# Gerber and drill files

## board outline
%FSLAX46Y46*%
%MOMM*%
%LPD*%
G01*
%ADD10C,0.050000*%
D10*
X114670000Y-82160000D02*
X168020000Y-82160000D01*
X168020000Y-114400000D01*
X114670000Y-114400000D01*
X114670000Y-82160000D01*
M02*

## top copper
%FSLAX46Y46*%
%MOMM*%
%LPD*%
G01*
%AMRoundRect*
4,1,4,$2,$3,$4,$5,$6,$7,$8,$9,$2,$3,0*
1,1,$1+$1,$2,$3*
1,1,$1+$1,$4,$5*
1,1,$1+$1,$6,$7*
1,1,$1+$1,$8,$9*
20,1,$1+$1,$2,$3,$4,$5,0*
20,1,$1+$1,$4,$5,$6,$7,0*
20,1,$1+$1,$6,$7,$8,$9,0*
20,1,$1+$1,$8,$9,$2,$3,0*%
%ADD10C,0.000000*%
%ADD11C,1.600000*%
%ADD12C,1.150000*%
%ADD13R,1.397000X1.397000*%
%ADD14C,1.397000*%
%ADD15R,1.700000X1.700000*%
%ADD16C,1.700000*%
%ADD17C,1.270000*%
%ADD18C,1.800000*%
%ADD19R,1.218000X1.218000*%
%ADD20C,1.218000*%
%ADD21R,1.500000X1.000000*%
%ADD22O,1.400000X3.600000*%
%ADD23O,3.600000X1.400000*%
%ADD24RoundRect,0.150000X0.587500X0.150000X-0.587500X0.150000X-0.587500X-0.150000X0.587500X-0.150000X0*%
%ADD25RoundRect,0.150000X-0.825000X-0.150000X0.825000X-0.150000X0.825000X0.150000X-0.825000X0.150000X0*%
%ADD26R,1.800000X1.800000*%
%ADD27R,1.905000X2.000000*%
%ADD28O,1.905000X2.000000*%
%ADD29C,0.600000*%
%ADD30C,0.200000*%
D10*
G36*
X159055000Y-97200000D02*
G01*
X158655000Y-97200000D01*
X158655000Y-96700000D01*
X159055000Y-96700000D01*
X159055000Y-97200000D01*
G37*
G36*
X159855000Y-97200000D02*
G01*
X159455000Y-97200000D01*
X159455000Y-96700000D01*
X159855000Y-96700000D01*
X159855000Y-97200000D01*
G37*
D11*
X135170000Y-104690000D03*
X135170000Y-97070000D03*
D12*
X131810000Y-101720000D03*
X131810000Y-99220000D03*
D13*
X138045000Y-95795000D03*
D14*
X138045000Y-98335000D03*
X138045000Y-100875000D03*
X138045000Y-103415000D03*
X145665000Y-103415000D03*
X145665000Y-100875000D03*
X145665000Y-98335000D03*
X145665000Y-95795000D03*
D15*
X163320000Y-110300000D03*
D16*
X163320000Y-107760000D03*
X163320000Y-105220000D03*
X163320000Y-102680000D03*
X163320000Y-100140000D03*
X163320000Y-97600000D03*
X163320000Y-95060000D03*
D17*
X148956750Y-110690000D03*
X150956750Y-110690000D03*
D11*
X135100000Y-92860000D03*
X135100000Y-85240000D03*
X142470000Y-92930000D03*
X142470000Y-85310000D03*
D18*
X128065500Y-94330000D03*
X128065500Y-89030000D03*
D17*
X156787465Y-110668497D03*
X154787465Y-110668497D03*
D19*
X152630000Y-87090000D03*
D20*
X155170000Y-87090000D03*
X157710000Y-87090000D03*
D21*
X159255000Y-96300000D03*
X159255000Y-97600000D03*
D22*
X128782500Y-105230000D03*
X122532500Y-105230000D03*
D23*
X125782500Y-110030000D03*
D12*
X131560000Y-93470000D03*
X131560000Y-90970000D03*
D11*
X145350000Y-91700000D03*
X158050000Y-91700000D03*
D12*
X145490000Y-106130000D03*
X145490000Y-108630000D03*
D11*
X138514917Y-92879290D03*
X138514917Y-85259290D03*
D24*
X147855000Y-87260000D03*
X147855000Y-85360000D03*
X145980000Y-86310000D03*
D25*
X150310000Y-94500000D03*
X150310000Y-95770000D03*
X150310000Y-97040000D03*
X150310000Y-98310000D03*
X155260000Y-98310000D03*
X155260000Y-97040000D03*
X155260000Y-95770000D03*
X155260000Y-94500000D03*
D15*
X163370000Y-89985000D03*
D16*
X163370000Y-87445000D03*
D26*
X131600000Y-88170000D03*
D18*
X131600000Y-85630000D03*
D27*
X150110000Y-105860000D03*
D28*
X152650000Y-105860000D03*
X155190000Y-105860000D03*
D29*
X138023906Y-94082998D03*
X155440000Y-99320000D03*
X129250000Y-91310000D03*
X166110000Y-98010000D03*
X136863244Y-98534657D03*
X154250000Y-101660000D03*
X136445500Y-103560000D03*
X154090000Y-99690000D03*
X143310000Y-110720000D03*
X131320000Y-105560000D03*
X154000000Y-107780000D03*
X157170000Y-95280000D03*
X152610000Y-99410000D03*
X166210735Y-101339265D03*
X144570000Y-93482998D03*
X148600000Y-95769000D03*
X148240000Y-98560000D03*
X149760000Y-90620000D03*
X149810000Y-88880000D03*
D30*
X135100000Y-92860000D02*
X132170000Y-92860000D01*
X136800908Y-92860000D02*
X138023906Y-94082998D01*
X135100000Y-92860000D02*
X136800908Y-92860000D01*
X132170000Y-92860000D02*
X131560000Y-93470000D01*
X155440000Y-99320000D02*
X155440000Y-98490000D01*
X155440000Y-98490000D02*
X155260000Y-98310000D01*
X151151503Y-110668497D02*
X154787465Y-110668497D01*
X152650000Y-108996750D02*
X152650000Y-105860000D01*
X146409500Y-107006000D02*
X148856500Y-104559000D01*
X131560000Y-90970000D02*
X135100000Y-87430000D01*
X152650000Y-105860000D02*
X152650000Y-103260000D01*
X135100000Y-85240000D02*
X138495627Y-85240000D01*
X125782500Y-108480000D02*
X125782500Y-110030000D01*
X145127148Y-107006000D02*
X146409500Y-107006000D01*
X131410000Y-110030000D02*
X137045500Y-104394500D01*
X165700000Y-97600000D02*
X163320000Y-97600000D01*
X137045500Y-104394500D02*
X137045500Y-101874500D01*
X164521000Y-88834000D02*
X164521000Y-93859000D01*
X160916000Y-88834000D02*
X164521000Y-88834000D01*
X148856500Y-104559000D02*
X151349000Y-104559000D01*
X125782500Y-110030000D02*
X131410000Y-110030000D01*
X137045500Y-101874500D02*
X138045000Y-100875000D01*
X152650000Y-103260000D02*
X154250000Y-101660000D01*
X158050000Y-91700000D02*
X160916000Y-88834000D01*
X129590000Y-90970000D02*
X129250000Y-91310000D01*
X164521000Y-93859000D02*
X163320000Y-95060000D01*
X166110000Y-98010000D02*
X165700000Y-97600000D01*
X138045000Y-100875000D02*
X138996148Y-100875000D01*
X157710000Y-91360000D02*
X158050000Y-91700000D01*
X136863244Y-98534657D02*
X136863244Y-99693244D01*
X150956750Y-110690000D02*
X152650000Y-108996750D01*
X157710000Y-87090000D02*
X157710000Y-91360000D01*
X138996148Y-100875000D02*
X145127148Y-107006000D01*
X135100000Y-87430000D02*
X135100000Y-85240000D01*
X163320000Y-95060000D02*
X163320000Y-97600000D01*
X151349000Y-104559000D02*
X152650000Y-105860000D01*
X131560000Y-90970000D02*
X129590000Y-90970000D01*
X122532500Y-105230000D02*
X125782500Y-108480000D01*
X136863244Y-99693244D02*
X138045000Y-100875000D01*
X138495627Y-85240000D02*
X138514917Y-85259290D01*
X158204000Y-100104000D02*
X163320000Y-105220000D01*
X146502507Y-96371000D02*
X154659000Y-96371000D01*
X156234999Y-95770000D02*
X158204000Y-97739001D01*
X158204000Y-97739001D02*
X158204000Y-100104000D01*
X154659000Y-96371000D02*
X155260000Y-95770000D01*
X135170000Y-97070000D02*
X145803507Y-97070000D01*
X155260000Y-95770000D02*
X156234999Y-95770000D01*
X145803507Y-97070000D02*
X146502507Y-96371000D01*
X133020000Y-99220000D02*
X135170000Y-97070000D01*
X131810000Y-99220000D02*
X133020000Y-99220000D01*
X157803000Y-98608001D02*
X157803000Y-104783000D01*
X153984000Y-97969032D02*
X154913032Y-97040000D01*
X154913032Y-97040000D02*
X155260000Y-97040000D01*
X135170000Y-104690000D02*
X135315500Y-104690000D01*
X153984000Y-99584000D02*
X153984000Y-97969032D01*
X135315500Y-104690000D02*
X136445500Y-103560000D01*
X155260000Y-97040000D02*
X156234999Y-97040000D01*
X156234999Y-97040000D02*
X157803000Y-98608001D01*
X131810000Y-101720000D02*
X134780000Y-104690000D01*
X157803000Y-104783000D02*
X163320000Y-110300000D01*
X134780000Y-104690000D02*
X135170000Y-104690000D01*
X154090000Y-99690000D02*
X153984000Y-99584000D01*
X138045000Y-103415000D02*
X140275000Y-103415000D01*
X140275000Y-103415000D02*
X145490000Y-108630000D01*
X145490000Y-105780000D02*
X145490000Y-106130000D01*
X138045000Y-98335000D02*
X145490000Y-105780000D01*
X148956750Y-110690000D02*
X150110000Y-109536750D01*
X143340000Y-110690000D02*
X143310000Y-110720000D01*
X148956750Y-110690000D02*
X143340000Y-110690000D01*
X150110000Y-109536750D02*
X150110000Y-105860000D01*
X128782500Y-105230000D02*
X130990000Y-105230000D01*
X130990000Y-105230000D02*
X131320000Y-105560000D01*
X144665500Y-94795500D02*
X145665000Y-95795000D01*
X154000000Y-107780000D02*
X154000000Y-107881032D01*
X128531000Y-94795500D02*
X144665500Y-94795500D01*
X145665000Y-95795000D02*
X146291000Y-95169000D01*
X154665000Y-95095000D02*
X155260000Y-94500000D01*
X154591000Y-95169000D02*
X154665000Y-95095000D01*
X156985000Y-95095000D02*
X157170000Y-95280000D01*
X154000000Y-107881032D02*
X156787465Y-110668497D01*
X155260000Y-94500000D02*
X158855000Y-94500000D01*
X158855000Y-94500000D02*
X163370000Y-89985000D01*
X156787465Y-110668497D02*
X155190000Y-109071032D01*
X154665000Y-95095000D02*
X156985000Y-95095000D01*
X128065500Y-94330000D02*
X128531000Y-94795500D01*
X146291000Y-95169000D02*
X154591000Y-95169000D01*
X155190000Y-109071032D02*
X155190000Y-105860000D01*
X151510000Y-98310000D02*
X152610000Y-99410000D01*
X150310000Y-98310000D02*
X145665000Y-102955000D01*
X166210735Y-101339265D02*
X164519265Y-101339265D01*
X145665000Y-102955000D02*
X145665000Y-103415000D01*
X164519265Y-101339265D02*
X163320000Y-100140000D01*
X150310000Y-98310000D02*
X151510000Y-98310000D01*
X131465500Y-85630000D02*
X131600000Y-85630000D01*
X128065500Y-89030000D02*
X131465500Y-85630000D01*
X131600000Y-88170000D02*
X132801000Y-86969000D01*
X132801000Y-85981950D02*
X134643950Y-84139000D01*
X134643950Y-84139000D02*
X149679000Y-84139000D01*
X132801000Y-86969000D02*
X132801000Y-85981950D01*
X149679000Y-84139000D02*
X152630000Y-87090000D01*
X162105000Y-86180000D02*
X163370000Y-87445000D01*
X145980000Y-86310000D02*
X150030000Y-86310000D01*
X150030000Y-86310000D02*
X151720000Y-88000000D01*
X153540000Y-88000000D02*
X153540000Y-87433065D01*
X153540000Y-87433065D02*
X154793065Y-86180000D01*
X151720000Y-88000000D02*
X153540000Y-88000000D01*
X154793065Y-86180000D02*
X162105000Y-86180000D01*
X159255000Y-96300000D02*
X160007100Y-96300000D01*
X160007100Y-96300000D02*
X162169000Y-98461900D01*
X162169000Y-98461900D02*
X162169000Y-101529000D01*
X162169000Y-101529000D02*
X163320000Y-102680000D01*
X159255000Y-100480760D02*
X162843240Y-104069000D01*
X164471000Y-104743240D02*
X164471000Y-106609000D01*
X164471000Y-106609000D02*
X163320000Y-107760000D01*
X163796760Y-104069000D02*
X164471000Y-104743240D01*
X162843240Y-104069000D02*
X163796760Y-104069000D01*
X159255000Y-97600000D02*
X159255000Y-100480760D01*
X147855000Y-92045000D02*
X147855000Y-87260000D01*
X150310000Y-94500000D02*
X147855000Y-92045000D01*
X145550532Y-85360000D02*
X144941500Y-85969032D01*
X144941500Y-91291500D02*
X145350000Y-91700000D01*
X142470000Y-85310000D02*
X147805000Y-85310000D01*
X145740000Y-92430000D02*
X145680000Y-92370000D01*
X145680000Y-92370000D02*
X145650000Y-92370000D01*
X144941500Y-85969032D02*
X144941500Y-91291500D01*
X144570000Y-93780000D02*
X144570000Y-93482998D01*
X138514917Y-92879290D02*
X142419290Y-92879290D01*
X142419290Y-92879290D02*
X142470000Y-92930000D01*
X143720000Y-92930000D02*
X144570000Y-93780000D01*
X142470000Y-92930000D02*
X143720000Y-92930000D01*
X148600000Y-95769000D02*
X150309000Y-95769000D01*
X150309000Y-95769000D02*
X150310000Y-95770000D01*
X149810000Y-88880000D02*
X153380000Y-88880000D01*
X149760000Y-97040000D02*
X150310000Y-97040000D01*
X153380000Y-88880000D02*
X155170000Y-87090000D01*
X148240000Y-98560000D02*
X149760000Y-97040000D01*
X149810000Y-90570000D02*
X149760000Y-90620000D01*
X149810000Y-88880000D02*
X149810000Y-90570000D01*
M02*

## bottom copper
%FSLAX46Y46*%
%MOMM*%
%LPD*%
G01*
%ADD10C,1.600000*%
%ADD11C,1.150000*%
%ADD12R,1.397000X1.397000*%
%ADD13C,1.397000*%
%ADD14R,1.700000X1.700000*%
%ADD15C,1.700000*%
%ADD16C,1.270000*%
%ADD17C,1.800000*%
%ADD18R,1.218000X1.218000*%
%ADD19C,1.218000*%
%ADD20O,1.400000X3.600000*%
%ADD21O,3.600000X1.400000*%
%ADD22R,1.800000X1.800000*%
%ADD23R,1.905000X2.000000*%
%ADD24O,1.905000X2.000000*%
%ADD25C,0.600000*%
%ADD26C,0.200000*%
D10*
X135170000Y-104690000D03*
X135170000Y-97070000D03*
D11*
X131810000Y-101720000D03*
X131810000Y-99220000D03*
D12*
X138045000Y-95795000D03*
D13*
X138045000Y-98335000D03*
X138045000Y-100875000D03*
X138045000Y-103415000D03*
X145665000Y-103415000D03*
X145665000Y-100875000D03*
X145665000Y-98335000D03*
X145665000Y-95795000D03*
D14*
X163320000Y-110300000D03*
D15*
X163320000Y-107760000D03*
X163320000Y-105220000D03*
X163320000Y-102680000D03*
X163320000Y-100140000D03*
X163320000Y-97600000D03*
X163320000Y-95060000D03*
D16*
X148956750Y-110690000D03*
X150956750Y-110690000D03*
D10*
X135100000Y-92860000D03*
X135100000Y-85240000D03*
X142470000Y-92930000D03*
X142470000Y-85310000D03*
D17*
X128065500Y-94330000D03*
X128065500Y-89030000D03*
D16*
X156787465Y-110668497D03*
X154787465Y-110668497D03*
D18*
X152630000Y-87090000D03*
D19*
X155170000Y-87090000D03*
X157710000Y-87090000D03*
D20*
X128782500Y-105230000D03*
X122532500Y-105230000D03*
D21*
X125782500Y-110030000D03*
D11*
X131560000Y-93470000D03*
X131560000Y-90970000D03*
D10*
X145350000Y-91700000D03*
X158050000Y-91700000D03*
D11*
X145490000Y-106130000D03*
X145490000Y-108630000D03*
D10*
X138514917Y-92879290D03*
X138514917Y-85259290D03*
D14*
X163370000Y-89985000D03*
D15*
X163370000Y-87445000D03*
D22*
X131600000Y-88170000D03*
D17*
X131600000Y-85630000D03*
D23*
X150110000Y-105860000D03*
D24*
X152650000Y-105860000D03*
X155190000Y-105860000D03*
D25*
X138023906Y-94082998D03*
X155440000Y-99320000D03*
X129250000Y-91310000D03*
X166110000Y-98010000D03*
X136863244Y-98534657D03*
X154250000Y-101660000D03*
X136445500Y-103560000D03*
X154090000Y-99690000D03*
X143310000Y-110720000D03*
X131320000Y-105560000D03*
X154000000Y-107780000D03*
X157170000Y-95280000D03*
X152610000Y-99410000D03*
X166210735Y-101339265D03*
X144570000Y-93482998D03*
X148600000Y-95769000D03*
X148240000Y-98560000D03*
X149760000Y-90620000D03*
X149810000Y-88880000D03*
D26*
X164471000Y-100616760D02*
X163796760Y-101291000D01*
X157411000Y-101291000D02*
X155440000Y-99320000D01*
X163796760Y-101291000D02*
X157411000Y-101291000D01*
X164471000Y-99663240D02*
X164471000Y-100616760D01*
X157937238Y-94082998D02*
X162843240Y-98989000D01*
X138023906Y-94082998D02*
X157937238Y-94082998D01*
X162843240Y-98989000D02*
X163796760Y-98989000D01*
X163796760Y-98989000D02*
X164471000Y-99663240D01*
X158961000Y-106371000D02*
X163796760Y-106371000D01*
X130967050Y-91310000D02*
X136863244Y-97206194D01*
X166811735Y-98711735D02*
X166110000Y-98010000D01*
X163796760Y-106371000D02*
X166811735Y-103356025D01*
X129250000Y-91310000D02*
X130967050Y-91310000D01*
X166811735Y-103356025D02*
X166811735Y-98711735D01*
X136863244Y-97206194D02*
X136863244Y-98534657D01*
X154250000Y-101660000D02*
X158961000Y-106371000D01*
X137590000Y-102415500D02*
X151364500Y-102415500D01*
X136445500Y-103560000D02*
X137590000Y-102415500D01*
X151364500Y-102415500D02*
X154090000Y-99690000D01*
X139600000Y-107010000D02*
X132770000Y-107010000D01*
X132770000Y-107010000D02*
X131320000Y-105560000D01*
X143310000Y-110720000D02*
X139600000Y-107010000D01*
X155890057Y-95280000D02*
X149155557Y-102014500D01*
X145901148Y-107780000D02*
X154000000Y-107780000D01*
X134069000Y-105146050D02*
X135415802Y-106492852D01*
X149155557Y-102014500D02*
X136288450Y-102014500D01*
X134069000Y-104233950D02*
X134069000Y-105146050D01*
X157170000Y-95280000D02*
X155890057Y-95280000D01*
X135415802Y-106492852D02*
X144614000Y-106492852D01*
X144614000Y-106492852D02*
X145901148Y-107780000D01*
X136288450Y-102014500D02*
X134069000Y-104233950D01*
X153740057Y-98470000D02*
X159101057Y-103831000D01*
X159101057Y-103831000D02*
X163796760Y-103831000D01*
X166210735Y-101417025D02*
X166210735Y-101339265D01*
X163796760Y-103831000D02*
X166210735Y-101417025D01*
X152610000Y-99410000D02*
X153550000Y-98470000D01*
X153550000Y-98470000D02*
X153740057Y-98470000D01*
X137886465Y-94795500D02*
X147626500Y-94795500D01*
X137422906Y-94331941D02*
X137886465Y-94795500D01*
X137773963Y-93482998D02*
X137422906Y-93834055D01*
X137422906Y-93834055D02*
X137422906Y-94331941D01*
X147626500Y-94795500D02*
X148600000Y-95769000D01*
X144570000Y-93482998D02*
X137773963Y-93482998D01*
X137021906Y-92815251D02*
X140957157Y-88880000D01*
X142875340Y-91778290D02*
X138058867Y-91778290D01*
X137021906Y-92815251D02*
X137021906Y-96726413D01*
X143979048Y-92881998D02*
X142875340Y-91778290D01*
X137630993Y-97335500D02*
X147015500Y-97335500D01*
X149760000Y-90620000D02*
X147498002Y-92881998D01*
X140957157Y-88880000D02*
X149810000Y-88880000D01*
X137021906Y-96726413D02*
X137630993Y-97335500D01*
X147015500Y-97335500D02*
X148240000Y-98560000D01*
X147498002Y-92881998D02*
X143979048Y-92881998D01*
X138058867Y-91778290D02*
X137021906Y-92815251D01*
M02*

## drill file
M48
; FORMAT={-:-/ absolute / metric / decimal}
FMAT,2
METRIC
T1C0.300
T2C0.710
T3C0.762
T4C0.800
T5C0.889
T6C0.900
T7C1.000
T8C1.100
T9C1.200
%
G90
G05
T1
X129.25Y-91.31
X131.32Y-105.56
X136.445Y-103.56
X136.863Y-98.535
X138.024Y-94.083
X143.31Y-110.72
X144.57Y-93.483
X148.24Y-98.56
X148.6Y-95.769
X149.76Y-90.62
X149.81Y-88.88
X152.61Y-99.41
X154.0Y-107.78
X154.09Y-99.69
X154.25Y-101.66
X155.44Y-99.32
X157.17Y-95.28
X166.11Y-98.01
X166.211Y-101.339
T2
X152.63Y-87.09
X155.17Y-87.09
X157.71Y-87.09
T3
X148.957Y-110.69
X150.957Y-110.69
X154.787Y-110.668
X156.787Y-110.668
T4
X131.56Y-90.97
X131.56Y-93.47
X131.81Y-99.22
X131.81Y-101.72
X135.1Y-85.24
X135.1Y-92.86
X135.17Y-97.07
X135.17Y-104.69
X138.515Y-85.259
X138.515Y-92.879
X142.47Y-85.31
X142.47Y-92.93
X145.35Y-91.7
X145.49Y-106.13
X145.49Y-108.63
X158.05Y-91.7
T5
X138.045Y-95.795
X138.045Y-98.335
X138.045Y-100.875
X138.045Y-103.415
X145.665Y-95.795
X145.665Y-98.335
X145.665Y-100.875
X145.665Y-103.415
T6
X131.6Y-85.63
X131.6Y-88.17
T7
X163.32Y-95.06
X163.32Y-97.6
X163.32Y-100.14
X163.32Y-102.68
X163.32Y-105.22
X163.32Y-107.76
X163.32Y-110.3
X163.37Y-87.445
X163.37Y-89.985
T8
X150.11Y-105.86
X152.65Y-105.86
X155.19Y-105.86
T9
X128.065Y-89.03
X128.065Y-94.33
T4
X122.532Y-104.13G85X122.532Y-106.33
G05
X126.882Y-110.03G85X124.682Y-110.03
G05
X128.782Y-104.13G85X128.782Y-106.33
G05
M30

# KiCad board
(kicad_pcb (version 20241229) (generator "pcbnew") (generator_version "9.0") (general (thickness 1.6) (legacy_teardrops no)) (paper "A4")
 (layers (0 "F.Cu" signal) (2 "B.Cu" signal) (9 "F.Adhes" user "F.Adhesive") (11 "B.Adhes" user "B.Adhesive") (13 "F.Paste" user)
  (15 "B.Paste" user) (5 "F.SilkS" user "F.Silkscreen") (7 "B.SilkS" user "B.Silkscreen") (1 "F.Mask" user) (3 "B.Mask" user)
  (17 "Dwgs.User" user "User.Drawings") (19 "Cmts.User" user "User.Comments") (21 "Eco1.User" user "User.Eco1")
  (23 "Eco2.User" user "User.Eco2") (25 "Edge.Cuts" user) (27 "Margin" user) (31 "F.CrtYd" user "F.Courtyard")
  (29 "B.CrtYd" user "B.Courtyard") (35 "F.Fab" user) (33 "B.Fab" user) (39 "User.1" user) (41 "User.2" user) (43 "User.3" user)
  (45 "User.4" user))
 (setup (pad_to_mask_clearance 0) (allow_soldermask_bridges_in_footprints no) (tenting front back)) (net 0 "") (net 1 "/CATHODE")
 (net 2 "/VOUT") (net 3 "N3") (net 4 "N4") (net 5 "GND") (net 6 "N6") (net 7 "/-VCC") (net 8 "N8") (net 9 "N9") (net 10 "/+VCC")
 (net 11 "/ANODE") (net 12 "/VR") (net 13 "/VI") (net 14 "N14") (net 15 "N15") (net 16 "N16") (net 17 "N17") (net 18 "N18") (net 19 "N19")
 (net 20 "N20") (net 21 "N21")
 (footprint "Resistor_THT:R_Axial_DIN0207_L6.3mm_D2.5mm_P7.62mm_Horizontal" (layer "F.Cu") (at 135.17 104.69 90)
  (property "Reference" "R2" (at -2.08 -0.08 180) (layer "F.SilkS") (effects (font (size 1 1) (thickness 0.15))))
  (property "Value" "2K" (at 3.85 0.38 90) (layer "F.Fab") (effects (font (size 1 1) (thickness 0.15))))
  (pad "1" thru_hole circle (at 0 0 90) (size 1.6 1.6) (drill 0.8) (layers "*.Cu" "*.Mask") (remove_unused_layers no) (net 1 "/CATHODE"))
  (pad "2" thru_hole circle (at 7.62 0 90) (size 1.6 1.6) (drill 0.8) (layers "*.Cu" "*.Mask") (remove_unused_layers no) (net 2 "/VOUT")))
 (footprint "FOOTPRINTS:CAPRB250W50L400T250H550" (layer "F.Cu") (at 131.81 100.47 90)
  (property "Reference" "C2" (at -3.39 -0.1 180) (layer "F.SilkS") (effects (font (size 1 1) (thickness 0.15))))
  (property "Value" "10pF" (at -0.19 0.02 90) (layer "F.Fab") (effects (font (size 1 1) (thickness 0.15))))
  (pad "1" thru_hole circle (at -1.25 0 90) (size 1.15 1.15) (drill 0.8) (layers "*.Cu" "*.Mask") (remove_unused_layers no)
   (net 1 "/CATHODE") (solder_mask_margin 0.102))
  (pad "2" thru_hole circle (at 1.25 0 90) (size 1.15 1.15) (drill 0.8) (layers "*.Cu" "*.Mask") (remove_unused_layers no) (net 2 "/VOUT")
   (solder_mask_margin 0.102)))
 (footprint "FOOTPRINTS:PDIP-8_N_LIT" (layer "F.Cu") (at 138.045 95.795)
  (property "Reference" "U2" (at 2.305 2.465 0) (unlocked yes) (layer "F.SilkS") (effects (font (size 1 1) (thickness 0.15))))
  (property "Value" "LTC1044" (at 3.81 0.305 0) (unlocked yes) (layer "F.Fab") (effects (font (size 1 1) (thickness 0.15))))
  (pad "1" thru_hole rect (at 0 0) (size 1.397 1.397) (drill 0.889) (layers "*.Cu" "*.Mask") (remove_unused_layers no) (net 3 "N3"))
  (pad "2" thru_hole circle (at 0 2.54) (size 1.397 1.397) (drill 0.889) (layers "*.Cu" "*.Mask") (remove_unused_layers no) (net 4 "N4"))
  (pad "3" thru_hole circle (at 0 5.08) (size 1.397 1.397) (drill 0.889) (layers "*.Cu" "*.Mask") (remove_unused_layers no) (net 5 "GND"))
  (pad "4" thru_hole circle (at 0 7.62) (size 1.397 1.397) (drill 0.889) (layers "*.Cu" "*.Mask") (remove_unused_layers no) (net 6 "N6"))
  (pad "5" thru_hole circle (at 7.62 7.62) (size 1.397 1.397) (drill 0.889) (layers "*.Cu" "*.Mask") (remove_unused_layers no)
   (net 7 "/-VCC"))
  (pad "6" thru_hole circle (at 7.62 5.08) (size 1.397 1.397) (drill 0.889) (layers "*.Cu" "*.Mask") (remove_unused_layers no) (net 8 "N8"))
  (pad "7" thru_hole circle (at 7.62 2.54) (size 1.397 1.397) (drill 0.889) (layers "*.Cu" "*.Mask") (remove_unused_layers no) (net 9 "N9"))
  (pad "8" thru_hole circle (at 7.62 0) (size 1.397 1.397) (drill 0.889) (layers "*.Cu" "*.Mask") (remove_unused_layers no) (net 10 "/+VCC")))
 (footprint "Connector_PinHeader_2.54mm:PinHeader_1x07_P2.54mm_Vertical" (layer "F.Cu") (at 163.32 110.3 180)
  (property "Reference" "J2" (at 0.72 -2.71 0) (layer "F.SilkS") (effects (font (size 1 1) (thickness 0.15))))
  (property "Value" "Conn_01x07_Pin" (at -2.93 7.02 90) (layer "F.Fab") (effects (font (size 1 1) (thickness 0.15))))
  (pad "1" thru_hole rect (at 0 0 180) (size 1.7 1.7) (drill 1) (layers "*.Cu" "*.Mask") (remove_unused_layers no) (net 1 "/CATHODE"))
  (pad "2" thru_hole circle (at 0 2.54 180) (size 1.7 1.7) (drill 1) (layers "*.Cu" "*.Mask") (remove_unused_layers no) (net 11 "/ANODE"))
  (pad "3" thru_hole circle (at 0 5.08 180) (size 1.7 1.7) (drill 1) (layers "*.Cu" "*.Mask") (remove_unused_layers no) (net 2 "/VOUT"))
  (pad "4" thru_hole circle (at 0 7.62 180) (size 1.7 1.7) (drill 1) (layers "*.Cu" "*.Mask") (remove_unused_layers no) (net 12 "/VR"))
  (pad "5" thru_hole circle (at 0 10.16 180) (size 1.7 1.7) (drill 1) (layers "*.Cu" "*.Mask") (remove_unused_layers no) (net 7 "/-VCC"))
  (pad "6" thru_hole circle (at 0 12.7 180) (size 1.7 1.7) (drill 1) (layers "*.Cu" "*.Mask") (remove_unused_layers no) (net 5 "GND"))
  (pad "7" thru_hole circle (at 0 15.24 180) (size 1.7 1.7) (drill 1) (layers "*.Cu" "*.Mask") (remove_unused_layers no) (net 5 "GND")))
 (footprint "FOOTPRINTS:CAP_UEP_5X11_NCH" (layer "F.Cu") (at 148.95675 110.69)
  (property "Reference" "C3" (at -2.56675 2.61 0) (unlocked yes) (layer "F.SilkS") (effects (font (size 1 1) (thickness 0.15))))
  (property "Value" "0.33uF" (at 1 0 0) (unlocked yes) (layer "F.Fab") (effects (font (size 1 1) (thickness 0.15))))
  (pad "1" thru_hole circle (at 0 0) (size 1.27 1.27) (drill 0.762) (layers "*.Cu" "*.Mask") (remove_unused_layers no) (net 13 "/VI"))
  (pad "2" thru_hole circle (at 2 0) (size 1.27 1.27) (drill 0.762) (layers "*.Cu" "*.Mask") (remove_unused_layers no) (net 5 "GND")))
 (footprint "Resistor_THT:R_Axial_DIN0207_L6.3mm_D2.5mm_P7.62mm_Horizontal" (layer "F.Cu") (at 135.1 92.86 90)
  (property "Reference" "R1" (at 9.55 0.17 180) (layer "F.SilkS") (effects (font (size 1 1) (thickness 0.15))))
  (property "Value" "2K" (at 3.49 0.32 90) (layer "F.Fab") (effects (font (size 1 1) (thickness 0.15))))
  (pad "1" thru_hole circle (at 0 0 90) (size 1.6 1.6) (drill 0.8) (layers "*.Cu" "*.Mask") (remove_unused_layers no) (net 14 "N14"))
  (pad "2" thru_hole circle (at 7.62 0 90) (size 1.6 1.6) (drill 0.8) (layers "*.Cu" "*.Mask") (remove_unused_layers no) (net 5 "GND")))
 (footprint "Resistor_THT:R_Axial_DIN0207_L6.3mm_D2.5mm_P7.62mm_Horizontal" (layer "F.Cu") (at 142.47 92.93 90)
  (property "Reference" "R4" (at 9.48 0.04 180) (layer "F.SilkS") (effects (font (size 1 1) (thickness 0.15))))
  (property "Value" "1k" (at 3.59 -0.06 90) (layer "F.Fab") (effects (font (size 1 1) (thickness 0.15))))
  (pad "1" thru_hole circle (at 0 0 90) (size 1.6 1.6) (drill 0.8) (layers "*.Cu" "*.Mask") (remove_unused_layers no) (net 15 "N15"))
  (pad "2" thru_hole circle (at 7.62 0 90) (size 1.6 1.6) (drill 0.8) (layers "*.Cu" "*.Mask") (remove_unused_layers no) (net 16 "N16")))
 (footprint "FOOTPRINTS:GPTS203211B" (layer "F.Cu") (at 128.1465 91.68)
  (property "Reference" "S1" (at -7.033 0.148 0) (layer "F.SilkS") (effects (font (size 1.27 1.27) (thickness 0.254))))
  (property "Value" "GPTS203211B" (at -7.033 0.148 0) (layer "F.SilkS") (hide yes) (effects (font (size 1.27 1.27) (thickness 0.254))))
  (pad "1" thru_hole circle (at -0.081 2.65) (size 1.8 1.8) (drill 1.2) (layers "*.Cu" "*.Mask") (remove_unused_layers no) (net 10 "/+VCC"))
  (pad "2" thru_hole circle (at -0.081 -2.65) (size 1.8 1.8) (drill 1.2) (layers "*.Cu" "*.Mask") (remove_unused_layers no) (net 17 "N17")))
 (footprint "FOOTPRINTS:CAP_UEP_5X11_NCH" (layer "F.Cu") (at 156.787465 110.668497 180)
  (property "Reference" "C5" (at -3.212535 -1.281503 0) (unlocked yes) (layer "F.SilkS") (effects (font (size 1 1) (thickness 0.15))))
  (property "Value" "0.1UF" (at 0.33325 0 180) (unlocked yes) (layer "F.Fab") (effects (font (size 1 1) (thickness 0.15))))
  (pad "1" thru_hole circle (at 0 0 180) (size 1.27 1.27) (drill 0.762) (layers "*.Cu" "*.Mask") (remove_unused_layers no) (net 10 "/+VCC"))
  (pad "2" thru_hole circle (at 2 0 180) (size 1.27 1.27) (drill 0.762) (layers "*.Cu" "*.Mask") (remove_unused_layers no) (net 5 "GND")))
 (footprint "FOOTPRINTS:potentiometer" (layer "F.Cu") (at 155.17 87.09)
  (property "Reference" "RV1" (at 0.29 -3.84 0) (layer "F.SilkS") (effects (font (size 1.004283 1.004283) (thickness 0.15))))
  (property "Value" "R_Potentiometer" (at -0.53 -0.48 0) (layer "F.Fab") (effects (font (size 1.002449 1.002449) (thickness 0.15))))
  (pad "1" thru_hole rect (at -2.54 0) (size 1.218 1.218) (drill 0.71) (layers "*.Cu" "*.Mask") (remove_unused_layers no) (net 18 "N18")
   (solder_mask_margin 0.102))
  (pad "2" thru_hole circle (at 0 0) (size 1.218 1.218) (drill 0.71) (layers "*.Cu" "*.Mask") (remove_unused_layers no) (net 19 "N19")
   (solder_mask_margin 0.102))
  (pad "3" thru_hole circle (at 2.54 0) (size 1.218 1.218) (drill 0.71) (layers "*.Cu" "*.Mask") (remove_unused_layers no) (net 5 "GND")
   (solder_mask_margin 0.102)))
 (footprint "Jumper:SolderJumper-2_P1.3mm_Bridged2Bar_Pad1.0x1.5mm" (layer "F.Cu") (at 159.255 96.95 -90)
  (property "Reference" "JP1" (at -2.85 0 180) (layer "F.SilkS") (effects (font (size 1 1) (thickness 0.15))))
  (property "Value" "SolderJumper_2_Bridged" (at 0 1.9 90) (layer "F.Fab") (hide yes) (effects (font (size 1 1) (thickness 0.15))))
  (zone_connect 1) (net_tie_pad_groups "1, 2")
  (fp_poly (pts (xy -0.25 0.2) (xy 0.25 0.2) (xy 0.25 0.6) (xy -0.25 0.6)) (stroke (width 0) (type solid)) (fill yes) (layer "F.Cu"))
  (fp_poly (pts (xy -0.25 -0.6) (xy 0.25 -0.6) (xy 0.25 -0.2) (xy -0.25 -0.2)) (stroke (width 0) (type solid)) (fill yes) (layer "F.Cu"))
  (pad "1" smd rect (at -0.65 0 270) (size 1 1.5) (layers "F.Cu" "F.Mask") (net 12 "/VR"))
  (pad "2" smd rect (at 0.65 0 270) (size 1 1.5) (layers "F.Cu" "F.Mask") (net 11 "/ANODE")))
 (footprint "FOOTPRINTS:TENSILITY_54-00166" (layer "F.Cu") (at 122.5325 105.23 -90)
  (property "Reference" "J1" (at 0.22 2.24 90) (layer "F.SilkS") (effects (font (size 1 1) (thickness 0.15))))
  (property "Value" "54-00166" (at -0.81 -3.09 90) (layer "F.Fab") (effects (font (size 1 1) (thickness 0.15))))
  (pad "A" thru_hole oval (at 0 -6.25 270) (size 3.6 1.4) (drill oval 3 0.8) (layers "*.Cu" "*.Mask") (remove_unused_layers no)
   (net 13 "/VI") (solder_mask_margin 0.102))
  (pad "B" thru_hole oval (at 0 0 270) (size 3.6 1.4) (drill oval 3 0.8) (layers "*.Cu" "*.Mask") (remove_unused_layers no) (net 5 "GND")
   (solder_mask_margin 0.102))
  (pad "C" thru_hole oval (at 4.8 -3.25 270) (size 1.4 3.6) (drill oval 0.8 3) (layers "*.Cu" "*.Mask") (remove_unused_layers no)
   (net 5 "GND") (solder_mask_margin 0.102)))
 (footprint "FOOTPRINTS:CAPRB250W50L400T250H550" (layer "F.Cu") (at 131.56 92.22 90)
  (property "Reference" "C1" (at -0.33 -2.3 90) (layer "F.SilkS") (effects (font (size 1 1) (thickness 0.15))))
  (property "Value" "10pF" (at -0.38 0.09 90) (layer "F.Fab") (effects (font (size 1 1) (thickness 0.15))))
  (pad "1" thru_hole circle (at -1.25 0 90) (size 1.15 1.15) (drill 0.8) (layers "*.Cu" "*.Mask") (remove_unused_layers no) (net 14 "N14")
   (solder_mask_margin 0.102))
  (pad "2" thru_hole circle (at 1.25 0 90) (size 1.15 1.15) (drill 0.8) (layers "*.Cu" "*.Mask") (remove_unused_layers no) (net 5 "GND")
   (solder_mask_margin 0.102)))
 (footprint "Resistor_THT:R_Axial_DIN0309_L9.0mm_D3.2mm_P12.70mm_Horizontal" (layer "F.Cu") (at 145.35 91.7)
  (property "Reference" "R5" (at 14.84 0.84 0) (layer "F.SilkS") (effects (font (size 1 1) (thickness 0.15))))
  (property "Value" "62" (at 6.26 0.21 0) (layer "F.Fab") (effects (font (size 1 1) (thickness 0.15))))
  (pad "1" thru_hole circle (at 0 0) (size 1.6 1.6) (drill 0.8) (layers "*.Cu" "*.Mask") (remove_unused_layers no) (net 16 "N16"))
  (pad "2" thru_hole circle (at 12.7 0) (size 1.6 1.6) (drill 0.8) (layers "*.Cu" "*.Mask") (remove_unused_layers no) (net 5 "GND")))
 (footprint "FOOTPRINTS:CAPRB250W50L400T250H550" (layer "F.Cu") (at 145.49 107.38 -90)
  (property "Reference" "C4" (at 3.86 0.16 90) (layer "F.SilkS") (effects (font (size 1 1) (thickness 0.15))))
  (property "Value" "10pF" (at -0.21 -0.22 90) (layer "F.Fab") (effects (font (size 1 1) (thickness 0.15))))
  (pad "1" thru_hole circle (at -1.25 0 270) (size 1.15 1.15) (drill 0.8) (layers "*.Cu" "*.Mask") (remove_unused_layers no) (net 4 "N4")
   (solder_mask_margin 0.102))
  (pad "2" thru_hole circle (at 1.25 0 270) (size 1.15 1.15) (drill 0.8) (layers "*.Cu" "*.Mask") (remove_unused_layers no) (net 6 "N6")
   (solder_mask_margin 0.102)))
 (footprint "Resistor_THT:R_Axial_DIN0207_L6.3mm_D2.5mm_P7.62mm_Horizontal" (layer "F.Cu") (at 138.514917 92.87929 90)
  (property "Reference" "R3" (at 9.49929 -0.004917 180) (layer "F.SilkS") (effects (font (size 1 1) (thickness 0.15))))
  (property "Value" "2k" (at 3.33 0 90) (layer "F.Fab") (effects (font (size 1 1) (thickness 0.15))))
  (pad "1" thru_hole circle (at 0 0 90) (size 1.6 1.6) (drill 0.8) (layers "*.Cu" "*.Mask") (remove_unused_layers no) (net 15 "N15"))
  (pad "2" thru_hole circle (at 7.62 0 90) (size 1.6 1.6) (drill 0.8) (layers "*.Cu" "*.Mask") (remove_unused_layers no) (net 5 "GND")))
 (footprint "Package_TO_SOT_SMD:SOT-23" (layer "F.Cu") (at 146.9175 86.31 180)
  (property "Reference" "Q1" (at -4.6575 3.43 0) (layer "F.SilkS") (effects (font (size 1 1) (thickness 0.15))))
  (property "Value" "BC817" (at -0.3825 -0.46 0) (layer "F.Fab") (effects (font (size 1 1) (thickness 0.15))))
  (pad "1" smd roundrect (at -0.9375 -0.95 180) (size 1.475 0.6) (layers "F.Cu" "F.Mask" "F.Paste") (roundrect_rratio 0.25) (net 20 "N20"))
  (pad "2" smd roundrect (at -0.9375 0.95 180) (size 1.475 0.6) (layers "F.Cu" "F.Mask" "F.Paste") (roundrect_rratio 0.25) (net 16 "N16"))
  (pad "3" smd roundrect (at 0.9375 0 180) (size 1.475 0.6) (layers "F.Cu" "F.Mask" "F.Paste") (roundrect_rratio 0.25) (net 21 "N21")))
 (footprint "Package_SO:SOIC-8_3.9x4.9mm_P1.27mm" (layer "F.Cu") (at 152.785 96.405)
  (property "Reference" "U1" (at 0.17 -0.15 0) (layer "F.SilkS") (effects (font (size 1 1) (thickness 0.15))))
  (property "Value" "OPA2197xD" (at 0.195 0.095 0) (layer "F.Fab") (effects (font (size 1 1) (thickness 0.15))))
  (pad "1" smd roundrect (at -2.475 -1.905) (size 1.95 0.6) (layers "F.Cu" "F.Mask" "F.Paste") (roundrect_rratio 0.25) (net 20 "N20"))
  (pad "2" smd roundrect (at -2.475 -0.635) (size 1.95 0.6) (layers "F.Cu" "F.Mask" "F.Paste") (roundrect_rratio 0.25) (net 15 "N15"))
  (pad "3" smd roundrect (at -2.475 0.635) (size 1.95 0.6) (layers "F.Cu" "F.Mask" "F.Paste") (roundrect_rratio 0.25) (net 19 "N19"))
  (pad "4" smd roundrect (at -2.475 1.905) (size 1.95 0.6) (layers "F.Cu" "F.Mask" "F.Paste") (roundrect_rratio 0.25) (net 7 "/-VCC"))
  (pad "5" smd roundrect (at 2.475 1.905) (size 1.95 0.6) (layers "F.Cu" "F.Mask" "F.Paste") (roundrect_rratio 0.25) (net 14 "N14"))
  (pad "6" smd roundrect (at 2.475 0.635) (size 1.95 0.6) (layers "F.Cu" "F.Mask" "F.Paste") (roundrect_rratio 0.25) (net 1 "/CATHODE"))
  (pad "7" smd roundrect (at 2.475 -0.635) (size 1.95 0.6) (layers "F.Cu" "F.Mask" "F.Paste") (roundrect_rratio 0.25) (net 2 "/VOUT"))
  (pad "8" smd roundrect (at 2.475 -1.905) (size 1.95 0.6) (layers "F.Cu" "F.Mask" "F.Paste") (roundrect_rratio 0.25) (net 10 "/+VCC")))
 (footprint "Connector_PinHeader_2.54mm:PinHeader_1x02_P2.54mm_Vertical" (layer "F.Cu") (at 163.37 89.985 180)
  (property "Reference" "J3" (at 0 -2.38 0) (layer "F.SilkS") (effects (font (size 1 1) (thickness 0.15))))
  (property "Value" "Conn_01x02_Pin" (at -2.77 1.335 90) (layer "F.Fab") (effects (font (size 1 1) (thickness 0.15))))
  (pad "1" thru_hole rect (at 0 0 180) (size 1.7 1.7) (drill 1) (layers "*.Cu" "*.Mask") (remove_unused_layers no) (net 10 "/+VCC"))
  (pad "2" thru_hole circle (at 0 2.54 180) (size 1.7 1.7) (drill 1) (layers "*.Cu" "*.Mask") (remove_unused_layers no) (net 21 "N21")))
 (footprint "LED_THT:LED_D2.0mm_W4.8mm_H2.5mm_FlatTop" (layer "F.Cu") (at 131.6 88.17 90)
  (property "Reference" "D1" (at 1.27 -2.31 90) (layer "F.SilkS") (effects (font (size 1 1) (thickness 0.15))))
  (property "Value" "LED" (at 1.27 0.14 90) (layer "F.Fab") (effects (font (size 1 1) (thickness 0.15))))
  (pad "1" thru_hole rect (at 0 0 90) (size 1.8 1.8) (drill 0.9) (layers "*.Cu" "*.Mask") (remove_unused_layers no) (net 18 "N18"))
  (pad "2" thru_hole circle (at 2.54 0 90) (size 1.8 1.8) (drill 0.9) (layers "*.Cu" "*.Mask") (remove_unused_layers no) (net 17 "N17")))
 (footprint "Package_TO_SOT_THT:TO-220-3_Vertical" (layer "F.Cu") (at 150.11 105.86)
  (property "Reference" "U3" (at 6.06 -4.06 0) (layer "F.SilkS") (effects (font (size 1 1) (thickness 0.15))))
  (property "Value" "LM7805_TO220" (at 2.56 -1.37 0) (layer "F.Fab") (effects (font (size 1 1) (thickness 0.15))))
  (pad "1" thru_hole rect (at 0 0) (size 1.905 2) (drill 1.1) (layers "*.Cu" "*.Mask") (remove_unused_layers no) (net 13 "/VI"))
  (pad "2" thru_hole oval (at 2.54 0) (size 1.905 2) (drill 1.1) (layers "*.Cu" "*.Mask") (remove_unused_layers no) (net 5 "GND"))
  (pad "3" thru_hole oval (at 5.08 0) (size 1.905 2) (drill 1.1) (layers "*.Cu" "*.Mask") (remove_unused_layers no) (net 10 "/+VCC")))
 (gr_rect (start 114.67 82.16) (end 168.02 114.4) (stroke (width 0.05) (type default)) (fill no) (layer "Edge.Cuts"))
 (segment (start 135.1 92.86) (end 132.17 92.86) (width 0.2) (layer "F.Cu") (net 14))
 (segment (start 136.800908 92.86) (end 138.023906 94.082998) (width 0.2) (layer "F.Cu") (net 14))
 (segment (start 135.1 92.86) (end 136.800908 92.86) (width 0.2) (layer "F.Cu") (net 14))
 (segment (start 132.17 92.86) (end 131.56 93.47) (width 0.2) (layer "F.Cu") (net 14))
 (segment (start 155.44 99.32) (end 155.44 98.49) (width 0.2) (layer "F.Cu") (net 14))
 (segment (start 155.44 98.49) (end 155.26 98.31) (width 0.2) (layer "F.Cu") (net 14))
 (via (at 138.023906 94.082998) (size 0.6) (drill 0.3) (layers "F.Cu" "B.Cu") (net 14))
 (via (at 155.44 99.32) (size 0.6) (drill 0.3) (layers "F.Cu" "B.Cu") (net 14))
 (segment (start 164.471 100.61676) (end 163.79676 101.291) (width 0.2) (layer "B.Cu") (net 14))
 (segment (start 157.411 101.291) (end 155.44 99.32) (width 0.2) (layer "B.Cu") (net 14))
 (segment (start 163.79676 101.291) (end 157.411 101.291) (width 0.2) (layer "B.Cu") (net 14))
 (segment (start 164.471 99.66324) (end 164.471 100.61676) (width 0.2) (layer "B.Cu") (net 14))
 (segment (start 157.937238 94.082998) (end 162.84324 98.989) (width 0.2) (layer "B.Cu") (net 14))
 (segment (start 138.023906 94.082998) (end 157.937238 94.082998) (width 0.2) (layer "B.Cu") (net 14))
 (segment (start 162.84324 98.989) (end 163.79676 98.989) (width 0.2) (layer "B.Cu") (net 14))
 (segment (start 163.79676 98.989) (end 164.471 99.66324) (width 0.2) (layer "B.Cu") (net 14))
 (segment (start 151.151503 110.668497) (end 154.787465 110.668497) (width 0.2) (layer "F.Cu") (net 5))
 (segment (start 152.65 108.99675) (end 152.65 105.86) (width 0.2) (layer "F.Cu") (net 5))
 (segment (start 146.4095 107.006) (end 148.8565 104.559) (width 0.2) (layer "F.Cu") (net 5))
 (segment (start 131.56 90.97) (end 135.1 87.43) (width 0.2) (layer "F.Cu") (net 5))
 (segment (start 152.65 105.86) (end 152.65 103.26) (width 0.2) (layer "F.Cu") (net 5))
 (segment (start 135.1 85.24) (end 138.495627 85.24) (width 0.2) (layer "F.Cu") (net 5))
 (segment (start 125.7825 108.48) (end 125.7825 110.03) (width 0.2) (layer "F.Cu") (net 5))
 (segment (start 145.127148 107.006) (end 146.4095 107.006) (width 0.2) (layer "F.Cu") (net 5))
 (segment (start 131.41 110.03) (end 137.0455 104.3945) (width 0.2) (layer "F.Cu") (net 5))
 (segment (start 165.7 97.6) (end 163.32 97.6) (width 0.2) (layer "F.Cu") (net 5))
 (segment (start 137.0455 104.3945) (end 137.0455 101.8745) (width 0.2) (layer "F.Cu") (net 5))
 (segment (start 164.521 88.834) (end 164.521 93.859) (width 0.2) (layer "F.Cu") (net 5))
 (segment (start 160.916 88.834) (end 164.521 88.834) (width 0.2) (layer "F.Cu") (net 5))
 (segment (start 148.8565 104.559) (end 151.349 104.559) (width 0.2) (layer "F.Cu") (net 5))
 (segment (start 125.7825 110.03) (end 131.41 110.03) (width 0.2) (layer "F.Cu") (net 5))
 (segment (start 137.0455 101.8745) (end 138.045 100.875) (width 0.2) (layer "F.Cu") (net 5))
 (segment (start 152.65 103.26) (end 154.25 101.66) (width 0.2) (layer "F.Cu") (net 5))
 (segment (start 158.05 91.7) (end 160.916 88.834) (width 0.2) (layer "F.Cu") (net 5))
 (segment (start 129.59 90.97) (end 129.25 91.31) (width 0.2) (layer "F.Cu") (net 5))
 (segment (start 164.521 93.859) (end 163.32 95.06) (width 0.2) (layer "F.Cu") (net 5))
 (segment (start 166.11 98.01) (end 165.7 97.6) (width 0.2) (layer "F.Cu") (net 5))
 (segment (start 138.045 100.875) (end 138.996148 100.875) (width 0.2) (layer "F.Cu") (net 5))
 (segment (start 157.71 91.36) (end 158.05 91.7) (width 0.2) (layer "F.Cu") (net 5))
 (segment (start 136.863244 98.534657) (end 136.863244 99.693244) (width 0.2) (layer "F.Cu") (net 5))
 (segment (start 150.95675 110.69) (end 152.65 108.99675) (width 0.2) (layer "F.Cu") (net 5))
 (segment (start 157.71 87.09) (end 157.71 91.36) (width 0.2) (layer "F.Cu") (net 5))
 (segment (start 138.996148 100.875) (end 145.127148 107.006) (width 0.2) (layer "F.Cu") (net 5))
 (segment (start 135.1 87.43) (end 135.1 85.24) (width 0.2) (layer "F.Cu") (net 5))
 (segment (start 163.32 95.06) (end 163.32 97.6) (width 0.2) (layer "F.Cu") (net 5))
 (segment (start 151.349 104.559) (end 152.65 105.86) (width 0.2) (layer "F.Cu") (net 5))
 (segment (start 131.56 90.97) (end 129.59 90.97) (width 0.2) (layer "F.Cu") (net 5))
 (segment (start 122.5325 105.23) (end 125.7825 108.48) (width 0.2) (layer "F.Cu") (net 5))
 (segment (start 136.863244 99.693244) (end 138.045 100.875) (width 0.2) (layer "F.Cu") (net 5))
 (segment (start 138.495627 85.24) (end 138.514917 85.25929) (width 0.2) (layer "F.Cu") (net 5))
 (via (at 129.25 91.31) (size 0.6) (drill 0.3) (layers "F.Cu" "B.Cu") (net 5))
 (via (at 166.11 98.01) (size 0.6) (drill 0.3) (layers "F.Cu" "B.Cu") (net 5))
 (via (at 136.863244 98.534657) (size 0.6) (drill 0.3) (layers "F.Cu" "B.Cu") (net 5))
 (via (at 154.25 101.66) (size 0.6) (drill 0.3) (layers "F.Cu" "B.Cu") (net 5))
 (segment (start 158.961 106.371) (end 163.79676 106.371) (width 0.2) (layer "B.Cu") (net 5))
 (segment (start 130.96705 91.31) (end 136.863244 97.206194) (width 0.2) (layer "B.Cu") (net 5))
 (segment (start 166.811735 98.711735) (end 166.11 98.01) (width 0.2) (layer "B.Cu") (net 5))
 (segment (start 163.79676 106.371) (end 166.811735 103.356025) (width 0.2) (layer "B.Cu") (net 5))
 (segment (start 129.25 91.31) (end 130.96705 91.31) (width 0.2) (layer "B.Cu") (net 5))
 (segment (start 166.811735 103.356025) (end 166.811735 98.711735) (width 0.2) (layer "B.Cu") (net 5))
 (segment (start 136.863244 97.206194) (end 136.863244 98.534657) (width 0.2) (layer "B.Cu") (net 5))
 (segment (start 154.25 101.66) (end 158.961 106.371) (width 0.2) (layer "B.Cu") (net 5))
 (segment (start 158.204 100.104) (end 163.32 105.22) (width 0.2) (layer "F.Cu") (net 2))
 (segment (start 146.502507 96.371) (end 154.659 96.371) (width 0.2) (layer "F.Cu") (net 2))
 (segment (start 156.234999 95.77) (end 158.204 97.739001) (width 0.2) (layer "F.Cu") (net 2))
 (segment (start 158.204 97.739001) (end 158.204 100.104) (width 0.2) (layer "F.Cu") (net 2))
 (segment (start 154.659 96.371) (end 155.26 95.77) (width 0.2) (layer "F.Cu") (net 2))
 (segment (start 135.17 97.07) (end 145.803507 97.07) (width 0.2) (layer "F.Cu") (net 2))
 (segment (start 155.26 95.77) (end 156.234999 95.77) (width 0.2) (layer "F.Cu") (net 2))
 (segment (start 145.803507 97.07) (end 146.502507 96.371) (width 0.2) (layer "F.Cu") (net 2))
 (segment (start 133.02 99.22) (end 135.17 97.07) (width 0.2) (layer "F.Cu") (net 2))
 (segment (start 131.81 99.22) (end 133.02 99.22) (width 0.2) (layer "F.Cu") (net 2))
 (segment (start 157.803 98.608001) (end 157.803 104.783) (width 0.2) (layer "F.Cu") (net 1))
 (segment (start 153.984 97.969032) (end 154.913032 97.04) (width 0.2) (layer "F.Cu") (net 1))
 (segment (start 154.913032 97.04) (end 155.26 97.04) (width 0.2) (layer "F.Cu") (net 1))
 (segment (start 135.17 104.69) (end 135.3155 104.69) (width 0.2) (layer "F.Cu") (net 1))
 (segment (start 153.984 99.584) (end 153.984 97.969032) (width 0.2) (layer "F.Cu") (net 1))
 (segment (start 135.3155 104.69) (end 136.4455 103.56) (width 0.2) (layer "F.Cu") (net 1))
 (segment (start 155.26 97.04) (end 156.234999 97.04) (width 0.2) (layer "F.Cu") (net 1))
 (segment (start 156.234999 97.04) (end 157.803 98.608001) (width 0.2) (layer "F.Cu") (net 1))
 (segment (start 131.81 101.72) (end 134.78 104.69) (width 0.2) (layer "F.Cu") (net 1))
 (segment (start 157.803 104.783) (end 163.32 110.3) (width 0.2) (layer "F.Cu") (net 1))
 (segment (start 134.78 104.69) (end 135.17 104.69) (width 0.2) (layer "F.Cu") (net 1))
 (segment (start 154.09 99.69) (end 153.984 99.584) (width 0.2) (layer "F.Cu") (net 1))
 (via (at 136.4455 103.56) (size 0.6) (drill 0.3) (layers "F.Cu" "B.Cu") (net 1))
 (via (at 154.09 99.69) (size 0.6) (drill 0.3) (layers "F.Cu" "B.Cu") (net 1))
 (segment (start 137.59 102.4155) (end 151.3645 102.4155) (width 0.2) (layer "B.Cu") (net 1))
 (segment (start 136.4455 103.56) (end 137.59 102.4155) (width 0.2) (layer "B.Cu") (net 1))
 (segment (start 151.3645 102.4155) (end 154.09 99.69) (width 0.2) (layer "B.Cu") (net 1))
 (segment (start 138.045 103.415) (end 140.275 103.415) (width 0.2) (layer "F.Cu") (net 6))
 (segment (start 140.275 103.415) (end 145.49 108.63) (width 0.2) (layer "F.Cu") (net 6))
 (segment (start 145.49 105.78) (end 145.49 106.13) (width 0.2) (layer "F.Cu") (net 4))
 (segment (start 138.045 98.335) (end 145.49 105.78) (width 0.2) (layer "F.Cu") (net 4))
 (segment (start 148.95675 110.69) (end 150.11 109.53675) (width 0.2) (layer "F.Cu") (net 13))
 (segment (start 143.34 110.69) (end 143.31 110.72) (width 0.2) (layer "F.Cu") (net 13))
 (segment (start 148.95675 110.69) (end 143.34 110.69) (width 0.2) (layer "F.Cu") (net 13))
 (segment (start 150.11 109.53675) (end 150.11 105.86) (width 0.2) (layer "F.Cu") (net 13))
 (segment (start 128.7825 105.23) (end 130.99 105.23) (width 0.2) (layer "F.Cu") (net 13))
 (segment (start 130.99 105.23) (end 131.32 105.56) (width 0.2) (layer "F.Cu") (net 13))
 (via (at 143.31 110.72) (size 0.6) (drill 0.3) (layers "F.Cu" "B.Cu") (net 13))
 (via (at 131.32 105.56) (size 0.6) (drill 0.3) (layers "F.Cu" "B.Cu") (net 13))
 (segment (start 139.6 107.01) (end 132.77 107.01) (width 0.2) (layer "B.Cu") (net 13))
 (segment (start 132.77 107.01) (end 131.32 105.56) (width 0.2) (layer "B.Cu") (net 13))
 (segment (start 143.31 110.72) (end 139.6 107.01) (width 0.2) (layer "B.Cu") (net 13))
 (segment (start 144.6655 94.7955) (end 145.665 95.795) (width 0.2) (layer "F.Cu") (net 10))
 (segment (start 154 107.78) (end 154 107.881032) (width 0.2) (layer "F.Cu") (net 10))
 (segment (start 128.531 94.7955) (end 144.6655 94.7955) (width 0.2) (layer "F.Cu") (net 10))
 (segment (start 145.665 95.795) (end 146.291 95.169) (width 0.2) (layer "F.Cu") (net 10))
 (segment (start 154.665 95.095) (end 155.26 94.5) (width 0.2) (layer "F.Cu") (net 10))
 (segment (start 154.591 95.169) (end 154.665 95.095) (width 0.2) (layer "F.Cu") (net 10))
 (segment (start 156.985 95.095) (end 157.17 95.28) (width 0.2) (layer "F.Cu") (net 10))
 (segment (start 154 107.881032) (end 156.787465 110.668497) (width 0.2) (layer "F.Cu") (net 10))
 (segment (start 155.26 94.5) (end 158.855 94.5) (width 0.2) (layer "F.Cu") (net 10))
 (segment (start 158.855 94.5) (end 163.37 89.985) (width 0.2) (layer "F.Cu") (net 10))
 (segment (start 156.787465 110.668497) (end 155.19 109.071032) (width 0.2) (layer "F.Cu") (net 10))
 (segment (start 154.665 95.095) (end 156.985 95.095) (width 0.2) (layer "F.Cu") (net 10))
 (segment (start 128.0655 94.33) (end 128.531 94.7955) (width 0.2) (layer "F.Cu") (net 10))
 (segment (start 146.291 95.169) (end 154.591 95.169) (width 0.2) (layer "F.Cu") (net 10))
 (segment (start 155.19 109.071032) (end 155.19 105.86) (width 0.2) (layer "F.Cu") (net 10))
 (via (at 154 107.78) (size 0.6) (drill 0.3) (layers "F.Cu" "B.Cu") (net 10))
 (via (at 157.17 95.28) (size 0.6) (drill 0.3) (layers "F.Cu" "B.Cu") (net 10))
 (segment (start 155.890057 95.28) (end 149.155557 102.0145) (width 0.2) (layer "B.Cu") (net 10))
 (segment (start 145.901148 107.78) (end 154 107.78) (width 0.2) (layer "B.Cu") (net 10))
 (segment (start 134.069 105.14605) (end 135.415802 106.492852) (width 0.2) (layer "B.Cu") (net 10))
 (segment (start 149.155557 102.0145) (end 136.28845 102.0145) (width 0.2) (layer "B.Cu") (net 10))
 (segment (start 134.069 104.23395) (end 134.069 105.14605) (width 0.2) (layer "B.Cu") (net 10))
 (segment (start 157.17 95.28) (end 155.890057 95.28) (width 0.2) (layer "B.Cu") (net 10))
 (segment (start 135.415802 106.492852) (end 144.614 106.492852) (width 0.2) (layer "B.Cu") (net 10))
 (segment (start 144.614 106.492852) (end 145.901148 107.78) (width 0.2) (layer "B.Cu") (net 10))
 (segment (start 136.28845 102.0145) (end 134.069 104.23395) (width 0.2) (layer "B.Cu") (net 10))
 (segment (start 151.51 98.31) (end 152.61 99.41) (width 0.2) (layer "F.Cu") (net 7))
 (segment (start 150.31 98.31) (end 145.665 102.955) (width 0.2) (layer "F.Cu") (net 7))
 (segment (start 166.210735 101.339265) (end 164.519265 101.339265) (width 0.2) (layer "F.Cu") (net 7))
 (segment (start 145.665 102.955) (end 145.665 103.415) (width 0.2) (layer "F.Cu") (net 7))
 (segment (start 164.519265 101.339265) (end 163.32 100.14) (width 0.2) (layer "F.Cu") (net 7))
 (segment (start 150.31 98.31) (end 151.51 98.31) (width 0.2) (layer "F.Cu") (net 7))
 (via (at 152.61 99.41) (size 0.6) (drill 0.3) (layers "F.Cu" "B.Cu") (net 7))
 (via (at 166.210735 101.339265) (size 0.6) (drill 0.3) (layers "F.Cu" "B.Cu") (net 7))
 (segment (start 153.740057 98.47) (end 159.101057 103.831) (width 0.2) (layer "B.Cu") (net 7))
 (segment (start 159.101057 103.831) (end 163.79676 103.831) (width 0.2) (layer "B.Cu") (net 7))
 (segment (start 166.210735 101.417025) (end 166.210735 101.339265) (width 0.2) (layer "B.Cu") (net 7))
 (segment (start 163.79676 103.831) (end 166.210735 101.417025) (width 0.2) (layer "B.Cu") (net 7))
 (segment (start 152.61 99.41) (end 153.55 98.47) (width 0.2) (layer "B.Cu") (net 7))
 (segment (start 153.55 98.47) (end 153.740057 98.47) (width 0.2) (layer "B.Cu") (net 7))
 (segment (start 131.4655 85.63) (end 131.6 85.63) (width 0.2) (layer "F.Cu") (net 17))
 (segment (start 128.0655 89.03) (end 131.4655 85.63) (width 0.2) (layer "F.Cu") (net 17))
 (segment (start 131.6 88.17) (end 132.801 86.969) (width 0.2) (layer "F.Cu") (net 18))
 (segment (start 132.801 85.98195) (end 134.64395 84.139) (width 0.2) (layer "F.Cu") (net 18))
 (segment (start 134.64395 84.139) (end 149.679 84.139) (width 0.2) (layer "F.Cu") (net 18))
 (segment (start 132.801 86.969) (end 132.801 85.98195) (width 0.2) (layer "F.Cu") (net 18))
 (segment (start 149.679 84.139) (end 152.63 87.09) (width 0.2) (layer "F.Cu") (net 18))
 (segment (start 162.105 86.18) (end 163.37 87.445) (width 0.2) (layer "F.Cu") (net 21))
 (segment (start 145.98 86.31) (end 150.03 86.31) (width 0.2) (layer "F.Cu") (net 21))
 (segment (start 150.03 86.31) (end 151.72 88) (width 0.2) (layer "F.Cu") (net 21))
 (segment (start 153.54 88) (end 153.54 87.433065) (width 0.2) (layer "F.Cu") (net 21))
 (segment (start 153.54 87.433065) (end 154.793065 86.18) (width 0.2) (layer "F.Cu") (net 21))
 (segment (start 151.72 88) (end 153.54 88) (width 0.2) (layer "F.Cu") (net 21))
 (segment (start 154.793065 86.18) (end 162.105 86.18) (width 0.2) (layer "F.Cu") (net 21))
 (segment (start 159.255 96.3) (end 160.0071 96.3) (width 0.2) (layer "F.Cu") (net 12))
 (segment (start 160.0071 96.3) (end 162.169 98.4619) (width 0.2) (layer "F.Cu") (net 12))
 (segment (start 162.169 98.4619) (end 162.169 101.529) (width 0.2) (layer "F.Cu") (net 12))
 (segment (start 162.169 101.529) (end 163.32 102.68) (width 0.2) (layer "F.Cu") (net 12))
 (segment (start 159.255 100.48076) (end 162.84324 104.069) (width 0.2) (layer "F.Cu") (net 11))
 (segment (start 164.471 104.74324) (end 164.471 106.609) (width 0.2) (layer "F.Cu") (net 11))
 (segment (start 164.471 106.609) (end 163.32 107.76) (width 0.2) (layer "F.Cu") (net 11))
 (segment (start 163.79676 104.069) (end 164.471 104.74324) (width 0.2) (layer "F.Cu") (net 11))
 (segment (start 162.84324 104.069) (end 163.79676 104.069) (width 0.2) (layer "F.Cu") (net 11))
 (segment (start 159.255 97.6) (end 159.255 100.48076) (width 0.2) (layer "F.Cu") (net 11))
 (segment (start 147.855 92.045) (end 147.855 87.26) (width 0.2) (layer "F.Cu") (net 20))
 (segment (start 150.31 94.5) (end 147.855 92.045) (width 0.2) (layer "F.Cu") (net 20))
 (segment (start 145.550532 85.36) (end 144.9415 85.969032) (width 0.2) (layer "F.Cu") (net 16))
 (segment (start 144.9415 91.2915) (end 145.35 91.7) (width 0.2) (layer "F.Cu") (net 16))
 (segment (start 142.47 85.31) (end 147.805 85.31) (width 0.2) (layer "F.Cu") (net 16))
 (segment (start 145.74 92.43) (end 145.68 92.37) (width 0.2) (layer "F.Cu") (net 16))
 (segment (start 145.68 92.37) (end 145.65 92.37) (width 0.2) (layer "F.Cu") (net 16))
 (segment (start 144.9415 85.969032) (end 144.9415 91.2915) (width 0.2) (layer "F.Cu") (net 16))
 (segment (start 144.57 93.78) (end 144.57 93.482998) (width 0.2) (layer "F.Cu") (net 15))
 (segment (start 138.514917 92.87929) (end 142.41929 92.87929) (width 0.2) (layer "F.Cu") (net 15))
 (segment (start 142.41929 92.87929) (end 142.47 92.93) (width 0.2) (layer "F.Cu") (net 15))
 (segment (start 143.72 92.93) (end 144.57 93.78) (width 0.2) (layer "F.Cu") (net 15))
 (segment (start 142.47 92.93) (end 143.72 92.93) (width 0.2) (layer "F.Cu") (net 15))
 (segment (start 148.6 95.769) (end 150.309 95.769) (width 0.2) (layer "F.Cu") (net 15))
 (segment (start 150.309 95.769) (end 150.31 95.77) (width 0.2) (layer "F.Cu") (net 15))
 (via (at 144.57 93.482998) (size 0.6) (drill 0.3) (layers "F.Cu" "B.Cu") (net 15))
 (via (at 148.6 95.769) (size 0.6) (drill 0.3) (layers "F.Cu" "B.Cu") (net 15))
 (segment (start 137.886465 94.7955) (end 147.6265 94.7955) (width 0.2) (layer "B.Cu") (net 15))
 (segment (start 137.422906 94.331941) (end 137.886465 94.7955) (width 0.2) (layer "B.Cu") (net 15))
 (segment (start 137.773963 93.482998) (end 137.422906 93.834055) (width 0.2) (layer "B.Cu") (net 15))
 (segment (start 137.422906 93.834055) (end 137.422906 94.331941) (width 0.2) (layer "B.Cu") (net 15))
 (segment (start 147.6265 94.7955) (end 148.6 95.769) (width 0.2) (layer "B.Cu") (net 15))
 (segment (start 144.57 93.482998) (end 137.773963 93.482998) (width 0.2) (layer "B.Cu") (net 15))
 (segment (start 149.81 88.88) (end 153.38 88.88) (width 0.2) (layer "F.Cu") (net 19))
 (segment (start 149.76 97.04) (end 150.31 97.04) (width 0.2) (layer "F.Cu") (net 19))
 (segment (start 153.38 88.88) (end 155.17 87.09) (width 0.2) (layer "F.Cu") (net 19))
 (segment (start 148.24 98.56) (end 149.76 97.04) (width 0.2) (layer "F.Cu") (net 19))
 (segment (start 149.81 90.57) (end 149.76 90.62) (width 0.2) (layer "F.Cu") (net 19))
 (segment (start 149.81 88.88) (end 149.81 90.57) (width 0.2) (layer "F.Cu") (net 19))
 (via (at 148.24 98.56) (size 0.6) (drill 0.3) (layers "F.Cu" "B.Cu") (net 19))
 (via (at 149.76 90.62) (size 0.6) (drill 0.3) (layers "F.Cu" "B.Cu") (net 19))
 (via (at 149.81 88.88) (size 0.6) (drill 0.3) (layers "F.Cu" "B.Cu") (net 19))
 (segment (start 137.021906 92.815251) (end 140.957157 88.88) (width 0.2) (layer "B.Cu") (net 19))
 (segment (start 142.87534 91.77829) (end 138.058867 91.77829) (width 0.2) (layer "B.Cu") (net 19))
 (segment (start 137.021906 92.815251) (end 137.021906 96.726413) (width 0.2) (layer "B.Cu") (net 19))
 (segment (start 143.979048 92.881998) (end 142.87534 91.77829) (width 0.2) (layer "B.Cu") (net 19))
 (segment (start 137.630993 97.3355) (end 147.0155 97.3355) (width 0.2) (layer "B.Cu") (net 19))
 (segment (start 149.76 90.62) (end 147.498002 92.881998) (width 0.2) (layer "B.Cu") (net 19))
 (segment (start 140.957157 88.88) (end 149.81 88.88) (width 0.2) (layer "B.Cu") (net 19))
 (segment (start 137.021906 96.726413) (end 137.630993 97.3355) (width 0.2) (layer "B.Cu") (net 19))
 (segment (start 147.0155 97.3355) (end 148.24 98.56) (width 0.2) (layer "B.Cu") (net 19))
 (segment (start 147.498002 92.881998) (end 143.979048 92.881998) (width 0.2) (layer "B.Cu") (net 19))
 (segment (start 138.058867 91.77829) (end 137.021906 92.815251) (width 0.2) (layer "B.Cu") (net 19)))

